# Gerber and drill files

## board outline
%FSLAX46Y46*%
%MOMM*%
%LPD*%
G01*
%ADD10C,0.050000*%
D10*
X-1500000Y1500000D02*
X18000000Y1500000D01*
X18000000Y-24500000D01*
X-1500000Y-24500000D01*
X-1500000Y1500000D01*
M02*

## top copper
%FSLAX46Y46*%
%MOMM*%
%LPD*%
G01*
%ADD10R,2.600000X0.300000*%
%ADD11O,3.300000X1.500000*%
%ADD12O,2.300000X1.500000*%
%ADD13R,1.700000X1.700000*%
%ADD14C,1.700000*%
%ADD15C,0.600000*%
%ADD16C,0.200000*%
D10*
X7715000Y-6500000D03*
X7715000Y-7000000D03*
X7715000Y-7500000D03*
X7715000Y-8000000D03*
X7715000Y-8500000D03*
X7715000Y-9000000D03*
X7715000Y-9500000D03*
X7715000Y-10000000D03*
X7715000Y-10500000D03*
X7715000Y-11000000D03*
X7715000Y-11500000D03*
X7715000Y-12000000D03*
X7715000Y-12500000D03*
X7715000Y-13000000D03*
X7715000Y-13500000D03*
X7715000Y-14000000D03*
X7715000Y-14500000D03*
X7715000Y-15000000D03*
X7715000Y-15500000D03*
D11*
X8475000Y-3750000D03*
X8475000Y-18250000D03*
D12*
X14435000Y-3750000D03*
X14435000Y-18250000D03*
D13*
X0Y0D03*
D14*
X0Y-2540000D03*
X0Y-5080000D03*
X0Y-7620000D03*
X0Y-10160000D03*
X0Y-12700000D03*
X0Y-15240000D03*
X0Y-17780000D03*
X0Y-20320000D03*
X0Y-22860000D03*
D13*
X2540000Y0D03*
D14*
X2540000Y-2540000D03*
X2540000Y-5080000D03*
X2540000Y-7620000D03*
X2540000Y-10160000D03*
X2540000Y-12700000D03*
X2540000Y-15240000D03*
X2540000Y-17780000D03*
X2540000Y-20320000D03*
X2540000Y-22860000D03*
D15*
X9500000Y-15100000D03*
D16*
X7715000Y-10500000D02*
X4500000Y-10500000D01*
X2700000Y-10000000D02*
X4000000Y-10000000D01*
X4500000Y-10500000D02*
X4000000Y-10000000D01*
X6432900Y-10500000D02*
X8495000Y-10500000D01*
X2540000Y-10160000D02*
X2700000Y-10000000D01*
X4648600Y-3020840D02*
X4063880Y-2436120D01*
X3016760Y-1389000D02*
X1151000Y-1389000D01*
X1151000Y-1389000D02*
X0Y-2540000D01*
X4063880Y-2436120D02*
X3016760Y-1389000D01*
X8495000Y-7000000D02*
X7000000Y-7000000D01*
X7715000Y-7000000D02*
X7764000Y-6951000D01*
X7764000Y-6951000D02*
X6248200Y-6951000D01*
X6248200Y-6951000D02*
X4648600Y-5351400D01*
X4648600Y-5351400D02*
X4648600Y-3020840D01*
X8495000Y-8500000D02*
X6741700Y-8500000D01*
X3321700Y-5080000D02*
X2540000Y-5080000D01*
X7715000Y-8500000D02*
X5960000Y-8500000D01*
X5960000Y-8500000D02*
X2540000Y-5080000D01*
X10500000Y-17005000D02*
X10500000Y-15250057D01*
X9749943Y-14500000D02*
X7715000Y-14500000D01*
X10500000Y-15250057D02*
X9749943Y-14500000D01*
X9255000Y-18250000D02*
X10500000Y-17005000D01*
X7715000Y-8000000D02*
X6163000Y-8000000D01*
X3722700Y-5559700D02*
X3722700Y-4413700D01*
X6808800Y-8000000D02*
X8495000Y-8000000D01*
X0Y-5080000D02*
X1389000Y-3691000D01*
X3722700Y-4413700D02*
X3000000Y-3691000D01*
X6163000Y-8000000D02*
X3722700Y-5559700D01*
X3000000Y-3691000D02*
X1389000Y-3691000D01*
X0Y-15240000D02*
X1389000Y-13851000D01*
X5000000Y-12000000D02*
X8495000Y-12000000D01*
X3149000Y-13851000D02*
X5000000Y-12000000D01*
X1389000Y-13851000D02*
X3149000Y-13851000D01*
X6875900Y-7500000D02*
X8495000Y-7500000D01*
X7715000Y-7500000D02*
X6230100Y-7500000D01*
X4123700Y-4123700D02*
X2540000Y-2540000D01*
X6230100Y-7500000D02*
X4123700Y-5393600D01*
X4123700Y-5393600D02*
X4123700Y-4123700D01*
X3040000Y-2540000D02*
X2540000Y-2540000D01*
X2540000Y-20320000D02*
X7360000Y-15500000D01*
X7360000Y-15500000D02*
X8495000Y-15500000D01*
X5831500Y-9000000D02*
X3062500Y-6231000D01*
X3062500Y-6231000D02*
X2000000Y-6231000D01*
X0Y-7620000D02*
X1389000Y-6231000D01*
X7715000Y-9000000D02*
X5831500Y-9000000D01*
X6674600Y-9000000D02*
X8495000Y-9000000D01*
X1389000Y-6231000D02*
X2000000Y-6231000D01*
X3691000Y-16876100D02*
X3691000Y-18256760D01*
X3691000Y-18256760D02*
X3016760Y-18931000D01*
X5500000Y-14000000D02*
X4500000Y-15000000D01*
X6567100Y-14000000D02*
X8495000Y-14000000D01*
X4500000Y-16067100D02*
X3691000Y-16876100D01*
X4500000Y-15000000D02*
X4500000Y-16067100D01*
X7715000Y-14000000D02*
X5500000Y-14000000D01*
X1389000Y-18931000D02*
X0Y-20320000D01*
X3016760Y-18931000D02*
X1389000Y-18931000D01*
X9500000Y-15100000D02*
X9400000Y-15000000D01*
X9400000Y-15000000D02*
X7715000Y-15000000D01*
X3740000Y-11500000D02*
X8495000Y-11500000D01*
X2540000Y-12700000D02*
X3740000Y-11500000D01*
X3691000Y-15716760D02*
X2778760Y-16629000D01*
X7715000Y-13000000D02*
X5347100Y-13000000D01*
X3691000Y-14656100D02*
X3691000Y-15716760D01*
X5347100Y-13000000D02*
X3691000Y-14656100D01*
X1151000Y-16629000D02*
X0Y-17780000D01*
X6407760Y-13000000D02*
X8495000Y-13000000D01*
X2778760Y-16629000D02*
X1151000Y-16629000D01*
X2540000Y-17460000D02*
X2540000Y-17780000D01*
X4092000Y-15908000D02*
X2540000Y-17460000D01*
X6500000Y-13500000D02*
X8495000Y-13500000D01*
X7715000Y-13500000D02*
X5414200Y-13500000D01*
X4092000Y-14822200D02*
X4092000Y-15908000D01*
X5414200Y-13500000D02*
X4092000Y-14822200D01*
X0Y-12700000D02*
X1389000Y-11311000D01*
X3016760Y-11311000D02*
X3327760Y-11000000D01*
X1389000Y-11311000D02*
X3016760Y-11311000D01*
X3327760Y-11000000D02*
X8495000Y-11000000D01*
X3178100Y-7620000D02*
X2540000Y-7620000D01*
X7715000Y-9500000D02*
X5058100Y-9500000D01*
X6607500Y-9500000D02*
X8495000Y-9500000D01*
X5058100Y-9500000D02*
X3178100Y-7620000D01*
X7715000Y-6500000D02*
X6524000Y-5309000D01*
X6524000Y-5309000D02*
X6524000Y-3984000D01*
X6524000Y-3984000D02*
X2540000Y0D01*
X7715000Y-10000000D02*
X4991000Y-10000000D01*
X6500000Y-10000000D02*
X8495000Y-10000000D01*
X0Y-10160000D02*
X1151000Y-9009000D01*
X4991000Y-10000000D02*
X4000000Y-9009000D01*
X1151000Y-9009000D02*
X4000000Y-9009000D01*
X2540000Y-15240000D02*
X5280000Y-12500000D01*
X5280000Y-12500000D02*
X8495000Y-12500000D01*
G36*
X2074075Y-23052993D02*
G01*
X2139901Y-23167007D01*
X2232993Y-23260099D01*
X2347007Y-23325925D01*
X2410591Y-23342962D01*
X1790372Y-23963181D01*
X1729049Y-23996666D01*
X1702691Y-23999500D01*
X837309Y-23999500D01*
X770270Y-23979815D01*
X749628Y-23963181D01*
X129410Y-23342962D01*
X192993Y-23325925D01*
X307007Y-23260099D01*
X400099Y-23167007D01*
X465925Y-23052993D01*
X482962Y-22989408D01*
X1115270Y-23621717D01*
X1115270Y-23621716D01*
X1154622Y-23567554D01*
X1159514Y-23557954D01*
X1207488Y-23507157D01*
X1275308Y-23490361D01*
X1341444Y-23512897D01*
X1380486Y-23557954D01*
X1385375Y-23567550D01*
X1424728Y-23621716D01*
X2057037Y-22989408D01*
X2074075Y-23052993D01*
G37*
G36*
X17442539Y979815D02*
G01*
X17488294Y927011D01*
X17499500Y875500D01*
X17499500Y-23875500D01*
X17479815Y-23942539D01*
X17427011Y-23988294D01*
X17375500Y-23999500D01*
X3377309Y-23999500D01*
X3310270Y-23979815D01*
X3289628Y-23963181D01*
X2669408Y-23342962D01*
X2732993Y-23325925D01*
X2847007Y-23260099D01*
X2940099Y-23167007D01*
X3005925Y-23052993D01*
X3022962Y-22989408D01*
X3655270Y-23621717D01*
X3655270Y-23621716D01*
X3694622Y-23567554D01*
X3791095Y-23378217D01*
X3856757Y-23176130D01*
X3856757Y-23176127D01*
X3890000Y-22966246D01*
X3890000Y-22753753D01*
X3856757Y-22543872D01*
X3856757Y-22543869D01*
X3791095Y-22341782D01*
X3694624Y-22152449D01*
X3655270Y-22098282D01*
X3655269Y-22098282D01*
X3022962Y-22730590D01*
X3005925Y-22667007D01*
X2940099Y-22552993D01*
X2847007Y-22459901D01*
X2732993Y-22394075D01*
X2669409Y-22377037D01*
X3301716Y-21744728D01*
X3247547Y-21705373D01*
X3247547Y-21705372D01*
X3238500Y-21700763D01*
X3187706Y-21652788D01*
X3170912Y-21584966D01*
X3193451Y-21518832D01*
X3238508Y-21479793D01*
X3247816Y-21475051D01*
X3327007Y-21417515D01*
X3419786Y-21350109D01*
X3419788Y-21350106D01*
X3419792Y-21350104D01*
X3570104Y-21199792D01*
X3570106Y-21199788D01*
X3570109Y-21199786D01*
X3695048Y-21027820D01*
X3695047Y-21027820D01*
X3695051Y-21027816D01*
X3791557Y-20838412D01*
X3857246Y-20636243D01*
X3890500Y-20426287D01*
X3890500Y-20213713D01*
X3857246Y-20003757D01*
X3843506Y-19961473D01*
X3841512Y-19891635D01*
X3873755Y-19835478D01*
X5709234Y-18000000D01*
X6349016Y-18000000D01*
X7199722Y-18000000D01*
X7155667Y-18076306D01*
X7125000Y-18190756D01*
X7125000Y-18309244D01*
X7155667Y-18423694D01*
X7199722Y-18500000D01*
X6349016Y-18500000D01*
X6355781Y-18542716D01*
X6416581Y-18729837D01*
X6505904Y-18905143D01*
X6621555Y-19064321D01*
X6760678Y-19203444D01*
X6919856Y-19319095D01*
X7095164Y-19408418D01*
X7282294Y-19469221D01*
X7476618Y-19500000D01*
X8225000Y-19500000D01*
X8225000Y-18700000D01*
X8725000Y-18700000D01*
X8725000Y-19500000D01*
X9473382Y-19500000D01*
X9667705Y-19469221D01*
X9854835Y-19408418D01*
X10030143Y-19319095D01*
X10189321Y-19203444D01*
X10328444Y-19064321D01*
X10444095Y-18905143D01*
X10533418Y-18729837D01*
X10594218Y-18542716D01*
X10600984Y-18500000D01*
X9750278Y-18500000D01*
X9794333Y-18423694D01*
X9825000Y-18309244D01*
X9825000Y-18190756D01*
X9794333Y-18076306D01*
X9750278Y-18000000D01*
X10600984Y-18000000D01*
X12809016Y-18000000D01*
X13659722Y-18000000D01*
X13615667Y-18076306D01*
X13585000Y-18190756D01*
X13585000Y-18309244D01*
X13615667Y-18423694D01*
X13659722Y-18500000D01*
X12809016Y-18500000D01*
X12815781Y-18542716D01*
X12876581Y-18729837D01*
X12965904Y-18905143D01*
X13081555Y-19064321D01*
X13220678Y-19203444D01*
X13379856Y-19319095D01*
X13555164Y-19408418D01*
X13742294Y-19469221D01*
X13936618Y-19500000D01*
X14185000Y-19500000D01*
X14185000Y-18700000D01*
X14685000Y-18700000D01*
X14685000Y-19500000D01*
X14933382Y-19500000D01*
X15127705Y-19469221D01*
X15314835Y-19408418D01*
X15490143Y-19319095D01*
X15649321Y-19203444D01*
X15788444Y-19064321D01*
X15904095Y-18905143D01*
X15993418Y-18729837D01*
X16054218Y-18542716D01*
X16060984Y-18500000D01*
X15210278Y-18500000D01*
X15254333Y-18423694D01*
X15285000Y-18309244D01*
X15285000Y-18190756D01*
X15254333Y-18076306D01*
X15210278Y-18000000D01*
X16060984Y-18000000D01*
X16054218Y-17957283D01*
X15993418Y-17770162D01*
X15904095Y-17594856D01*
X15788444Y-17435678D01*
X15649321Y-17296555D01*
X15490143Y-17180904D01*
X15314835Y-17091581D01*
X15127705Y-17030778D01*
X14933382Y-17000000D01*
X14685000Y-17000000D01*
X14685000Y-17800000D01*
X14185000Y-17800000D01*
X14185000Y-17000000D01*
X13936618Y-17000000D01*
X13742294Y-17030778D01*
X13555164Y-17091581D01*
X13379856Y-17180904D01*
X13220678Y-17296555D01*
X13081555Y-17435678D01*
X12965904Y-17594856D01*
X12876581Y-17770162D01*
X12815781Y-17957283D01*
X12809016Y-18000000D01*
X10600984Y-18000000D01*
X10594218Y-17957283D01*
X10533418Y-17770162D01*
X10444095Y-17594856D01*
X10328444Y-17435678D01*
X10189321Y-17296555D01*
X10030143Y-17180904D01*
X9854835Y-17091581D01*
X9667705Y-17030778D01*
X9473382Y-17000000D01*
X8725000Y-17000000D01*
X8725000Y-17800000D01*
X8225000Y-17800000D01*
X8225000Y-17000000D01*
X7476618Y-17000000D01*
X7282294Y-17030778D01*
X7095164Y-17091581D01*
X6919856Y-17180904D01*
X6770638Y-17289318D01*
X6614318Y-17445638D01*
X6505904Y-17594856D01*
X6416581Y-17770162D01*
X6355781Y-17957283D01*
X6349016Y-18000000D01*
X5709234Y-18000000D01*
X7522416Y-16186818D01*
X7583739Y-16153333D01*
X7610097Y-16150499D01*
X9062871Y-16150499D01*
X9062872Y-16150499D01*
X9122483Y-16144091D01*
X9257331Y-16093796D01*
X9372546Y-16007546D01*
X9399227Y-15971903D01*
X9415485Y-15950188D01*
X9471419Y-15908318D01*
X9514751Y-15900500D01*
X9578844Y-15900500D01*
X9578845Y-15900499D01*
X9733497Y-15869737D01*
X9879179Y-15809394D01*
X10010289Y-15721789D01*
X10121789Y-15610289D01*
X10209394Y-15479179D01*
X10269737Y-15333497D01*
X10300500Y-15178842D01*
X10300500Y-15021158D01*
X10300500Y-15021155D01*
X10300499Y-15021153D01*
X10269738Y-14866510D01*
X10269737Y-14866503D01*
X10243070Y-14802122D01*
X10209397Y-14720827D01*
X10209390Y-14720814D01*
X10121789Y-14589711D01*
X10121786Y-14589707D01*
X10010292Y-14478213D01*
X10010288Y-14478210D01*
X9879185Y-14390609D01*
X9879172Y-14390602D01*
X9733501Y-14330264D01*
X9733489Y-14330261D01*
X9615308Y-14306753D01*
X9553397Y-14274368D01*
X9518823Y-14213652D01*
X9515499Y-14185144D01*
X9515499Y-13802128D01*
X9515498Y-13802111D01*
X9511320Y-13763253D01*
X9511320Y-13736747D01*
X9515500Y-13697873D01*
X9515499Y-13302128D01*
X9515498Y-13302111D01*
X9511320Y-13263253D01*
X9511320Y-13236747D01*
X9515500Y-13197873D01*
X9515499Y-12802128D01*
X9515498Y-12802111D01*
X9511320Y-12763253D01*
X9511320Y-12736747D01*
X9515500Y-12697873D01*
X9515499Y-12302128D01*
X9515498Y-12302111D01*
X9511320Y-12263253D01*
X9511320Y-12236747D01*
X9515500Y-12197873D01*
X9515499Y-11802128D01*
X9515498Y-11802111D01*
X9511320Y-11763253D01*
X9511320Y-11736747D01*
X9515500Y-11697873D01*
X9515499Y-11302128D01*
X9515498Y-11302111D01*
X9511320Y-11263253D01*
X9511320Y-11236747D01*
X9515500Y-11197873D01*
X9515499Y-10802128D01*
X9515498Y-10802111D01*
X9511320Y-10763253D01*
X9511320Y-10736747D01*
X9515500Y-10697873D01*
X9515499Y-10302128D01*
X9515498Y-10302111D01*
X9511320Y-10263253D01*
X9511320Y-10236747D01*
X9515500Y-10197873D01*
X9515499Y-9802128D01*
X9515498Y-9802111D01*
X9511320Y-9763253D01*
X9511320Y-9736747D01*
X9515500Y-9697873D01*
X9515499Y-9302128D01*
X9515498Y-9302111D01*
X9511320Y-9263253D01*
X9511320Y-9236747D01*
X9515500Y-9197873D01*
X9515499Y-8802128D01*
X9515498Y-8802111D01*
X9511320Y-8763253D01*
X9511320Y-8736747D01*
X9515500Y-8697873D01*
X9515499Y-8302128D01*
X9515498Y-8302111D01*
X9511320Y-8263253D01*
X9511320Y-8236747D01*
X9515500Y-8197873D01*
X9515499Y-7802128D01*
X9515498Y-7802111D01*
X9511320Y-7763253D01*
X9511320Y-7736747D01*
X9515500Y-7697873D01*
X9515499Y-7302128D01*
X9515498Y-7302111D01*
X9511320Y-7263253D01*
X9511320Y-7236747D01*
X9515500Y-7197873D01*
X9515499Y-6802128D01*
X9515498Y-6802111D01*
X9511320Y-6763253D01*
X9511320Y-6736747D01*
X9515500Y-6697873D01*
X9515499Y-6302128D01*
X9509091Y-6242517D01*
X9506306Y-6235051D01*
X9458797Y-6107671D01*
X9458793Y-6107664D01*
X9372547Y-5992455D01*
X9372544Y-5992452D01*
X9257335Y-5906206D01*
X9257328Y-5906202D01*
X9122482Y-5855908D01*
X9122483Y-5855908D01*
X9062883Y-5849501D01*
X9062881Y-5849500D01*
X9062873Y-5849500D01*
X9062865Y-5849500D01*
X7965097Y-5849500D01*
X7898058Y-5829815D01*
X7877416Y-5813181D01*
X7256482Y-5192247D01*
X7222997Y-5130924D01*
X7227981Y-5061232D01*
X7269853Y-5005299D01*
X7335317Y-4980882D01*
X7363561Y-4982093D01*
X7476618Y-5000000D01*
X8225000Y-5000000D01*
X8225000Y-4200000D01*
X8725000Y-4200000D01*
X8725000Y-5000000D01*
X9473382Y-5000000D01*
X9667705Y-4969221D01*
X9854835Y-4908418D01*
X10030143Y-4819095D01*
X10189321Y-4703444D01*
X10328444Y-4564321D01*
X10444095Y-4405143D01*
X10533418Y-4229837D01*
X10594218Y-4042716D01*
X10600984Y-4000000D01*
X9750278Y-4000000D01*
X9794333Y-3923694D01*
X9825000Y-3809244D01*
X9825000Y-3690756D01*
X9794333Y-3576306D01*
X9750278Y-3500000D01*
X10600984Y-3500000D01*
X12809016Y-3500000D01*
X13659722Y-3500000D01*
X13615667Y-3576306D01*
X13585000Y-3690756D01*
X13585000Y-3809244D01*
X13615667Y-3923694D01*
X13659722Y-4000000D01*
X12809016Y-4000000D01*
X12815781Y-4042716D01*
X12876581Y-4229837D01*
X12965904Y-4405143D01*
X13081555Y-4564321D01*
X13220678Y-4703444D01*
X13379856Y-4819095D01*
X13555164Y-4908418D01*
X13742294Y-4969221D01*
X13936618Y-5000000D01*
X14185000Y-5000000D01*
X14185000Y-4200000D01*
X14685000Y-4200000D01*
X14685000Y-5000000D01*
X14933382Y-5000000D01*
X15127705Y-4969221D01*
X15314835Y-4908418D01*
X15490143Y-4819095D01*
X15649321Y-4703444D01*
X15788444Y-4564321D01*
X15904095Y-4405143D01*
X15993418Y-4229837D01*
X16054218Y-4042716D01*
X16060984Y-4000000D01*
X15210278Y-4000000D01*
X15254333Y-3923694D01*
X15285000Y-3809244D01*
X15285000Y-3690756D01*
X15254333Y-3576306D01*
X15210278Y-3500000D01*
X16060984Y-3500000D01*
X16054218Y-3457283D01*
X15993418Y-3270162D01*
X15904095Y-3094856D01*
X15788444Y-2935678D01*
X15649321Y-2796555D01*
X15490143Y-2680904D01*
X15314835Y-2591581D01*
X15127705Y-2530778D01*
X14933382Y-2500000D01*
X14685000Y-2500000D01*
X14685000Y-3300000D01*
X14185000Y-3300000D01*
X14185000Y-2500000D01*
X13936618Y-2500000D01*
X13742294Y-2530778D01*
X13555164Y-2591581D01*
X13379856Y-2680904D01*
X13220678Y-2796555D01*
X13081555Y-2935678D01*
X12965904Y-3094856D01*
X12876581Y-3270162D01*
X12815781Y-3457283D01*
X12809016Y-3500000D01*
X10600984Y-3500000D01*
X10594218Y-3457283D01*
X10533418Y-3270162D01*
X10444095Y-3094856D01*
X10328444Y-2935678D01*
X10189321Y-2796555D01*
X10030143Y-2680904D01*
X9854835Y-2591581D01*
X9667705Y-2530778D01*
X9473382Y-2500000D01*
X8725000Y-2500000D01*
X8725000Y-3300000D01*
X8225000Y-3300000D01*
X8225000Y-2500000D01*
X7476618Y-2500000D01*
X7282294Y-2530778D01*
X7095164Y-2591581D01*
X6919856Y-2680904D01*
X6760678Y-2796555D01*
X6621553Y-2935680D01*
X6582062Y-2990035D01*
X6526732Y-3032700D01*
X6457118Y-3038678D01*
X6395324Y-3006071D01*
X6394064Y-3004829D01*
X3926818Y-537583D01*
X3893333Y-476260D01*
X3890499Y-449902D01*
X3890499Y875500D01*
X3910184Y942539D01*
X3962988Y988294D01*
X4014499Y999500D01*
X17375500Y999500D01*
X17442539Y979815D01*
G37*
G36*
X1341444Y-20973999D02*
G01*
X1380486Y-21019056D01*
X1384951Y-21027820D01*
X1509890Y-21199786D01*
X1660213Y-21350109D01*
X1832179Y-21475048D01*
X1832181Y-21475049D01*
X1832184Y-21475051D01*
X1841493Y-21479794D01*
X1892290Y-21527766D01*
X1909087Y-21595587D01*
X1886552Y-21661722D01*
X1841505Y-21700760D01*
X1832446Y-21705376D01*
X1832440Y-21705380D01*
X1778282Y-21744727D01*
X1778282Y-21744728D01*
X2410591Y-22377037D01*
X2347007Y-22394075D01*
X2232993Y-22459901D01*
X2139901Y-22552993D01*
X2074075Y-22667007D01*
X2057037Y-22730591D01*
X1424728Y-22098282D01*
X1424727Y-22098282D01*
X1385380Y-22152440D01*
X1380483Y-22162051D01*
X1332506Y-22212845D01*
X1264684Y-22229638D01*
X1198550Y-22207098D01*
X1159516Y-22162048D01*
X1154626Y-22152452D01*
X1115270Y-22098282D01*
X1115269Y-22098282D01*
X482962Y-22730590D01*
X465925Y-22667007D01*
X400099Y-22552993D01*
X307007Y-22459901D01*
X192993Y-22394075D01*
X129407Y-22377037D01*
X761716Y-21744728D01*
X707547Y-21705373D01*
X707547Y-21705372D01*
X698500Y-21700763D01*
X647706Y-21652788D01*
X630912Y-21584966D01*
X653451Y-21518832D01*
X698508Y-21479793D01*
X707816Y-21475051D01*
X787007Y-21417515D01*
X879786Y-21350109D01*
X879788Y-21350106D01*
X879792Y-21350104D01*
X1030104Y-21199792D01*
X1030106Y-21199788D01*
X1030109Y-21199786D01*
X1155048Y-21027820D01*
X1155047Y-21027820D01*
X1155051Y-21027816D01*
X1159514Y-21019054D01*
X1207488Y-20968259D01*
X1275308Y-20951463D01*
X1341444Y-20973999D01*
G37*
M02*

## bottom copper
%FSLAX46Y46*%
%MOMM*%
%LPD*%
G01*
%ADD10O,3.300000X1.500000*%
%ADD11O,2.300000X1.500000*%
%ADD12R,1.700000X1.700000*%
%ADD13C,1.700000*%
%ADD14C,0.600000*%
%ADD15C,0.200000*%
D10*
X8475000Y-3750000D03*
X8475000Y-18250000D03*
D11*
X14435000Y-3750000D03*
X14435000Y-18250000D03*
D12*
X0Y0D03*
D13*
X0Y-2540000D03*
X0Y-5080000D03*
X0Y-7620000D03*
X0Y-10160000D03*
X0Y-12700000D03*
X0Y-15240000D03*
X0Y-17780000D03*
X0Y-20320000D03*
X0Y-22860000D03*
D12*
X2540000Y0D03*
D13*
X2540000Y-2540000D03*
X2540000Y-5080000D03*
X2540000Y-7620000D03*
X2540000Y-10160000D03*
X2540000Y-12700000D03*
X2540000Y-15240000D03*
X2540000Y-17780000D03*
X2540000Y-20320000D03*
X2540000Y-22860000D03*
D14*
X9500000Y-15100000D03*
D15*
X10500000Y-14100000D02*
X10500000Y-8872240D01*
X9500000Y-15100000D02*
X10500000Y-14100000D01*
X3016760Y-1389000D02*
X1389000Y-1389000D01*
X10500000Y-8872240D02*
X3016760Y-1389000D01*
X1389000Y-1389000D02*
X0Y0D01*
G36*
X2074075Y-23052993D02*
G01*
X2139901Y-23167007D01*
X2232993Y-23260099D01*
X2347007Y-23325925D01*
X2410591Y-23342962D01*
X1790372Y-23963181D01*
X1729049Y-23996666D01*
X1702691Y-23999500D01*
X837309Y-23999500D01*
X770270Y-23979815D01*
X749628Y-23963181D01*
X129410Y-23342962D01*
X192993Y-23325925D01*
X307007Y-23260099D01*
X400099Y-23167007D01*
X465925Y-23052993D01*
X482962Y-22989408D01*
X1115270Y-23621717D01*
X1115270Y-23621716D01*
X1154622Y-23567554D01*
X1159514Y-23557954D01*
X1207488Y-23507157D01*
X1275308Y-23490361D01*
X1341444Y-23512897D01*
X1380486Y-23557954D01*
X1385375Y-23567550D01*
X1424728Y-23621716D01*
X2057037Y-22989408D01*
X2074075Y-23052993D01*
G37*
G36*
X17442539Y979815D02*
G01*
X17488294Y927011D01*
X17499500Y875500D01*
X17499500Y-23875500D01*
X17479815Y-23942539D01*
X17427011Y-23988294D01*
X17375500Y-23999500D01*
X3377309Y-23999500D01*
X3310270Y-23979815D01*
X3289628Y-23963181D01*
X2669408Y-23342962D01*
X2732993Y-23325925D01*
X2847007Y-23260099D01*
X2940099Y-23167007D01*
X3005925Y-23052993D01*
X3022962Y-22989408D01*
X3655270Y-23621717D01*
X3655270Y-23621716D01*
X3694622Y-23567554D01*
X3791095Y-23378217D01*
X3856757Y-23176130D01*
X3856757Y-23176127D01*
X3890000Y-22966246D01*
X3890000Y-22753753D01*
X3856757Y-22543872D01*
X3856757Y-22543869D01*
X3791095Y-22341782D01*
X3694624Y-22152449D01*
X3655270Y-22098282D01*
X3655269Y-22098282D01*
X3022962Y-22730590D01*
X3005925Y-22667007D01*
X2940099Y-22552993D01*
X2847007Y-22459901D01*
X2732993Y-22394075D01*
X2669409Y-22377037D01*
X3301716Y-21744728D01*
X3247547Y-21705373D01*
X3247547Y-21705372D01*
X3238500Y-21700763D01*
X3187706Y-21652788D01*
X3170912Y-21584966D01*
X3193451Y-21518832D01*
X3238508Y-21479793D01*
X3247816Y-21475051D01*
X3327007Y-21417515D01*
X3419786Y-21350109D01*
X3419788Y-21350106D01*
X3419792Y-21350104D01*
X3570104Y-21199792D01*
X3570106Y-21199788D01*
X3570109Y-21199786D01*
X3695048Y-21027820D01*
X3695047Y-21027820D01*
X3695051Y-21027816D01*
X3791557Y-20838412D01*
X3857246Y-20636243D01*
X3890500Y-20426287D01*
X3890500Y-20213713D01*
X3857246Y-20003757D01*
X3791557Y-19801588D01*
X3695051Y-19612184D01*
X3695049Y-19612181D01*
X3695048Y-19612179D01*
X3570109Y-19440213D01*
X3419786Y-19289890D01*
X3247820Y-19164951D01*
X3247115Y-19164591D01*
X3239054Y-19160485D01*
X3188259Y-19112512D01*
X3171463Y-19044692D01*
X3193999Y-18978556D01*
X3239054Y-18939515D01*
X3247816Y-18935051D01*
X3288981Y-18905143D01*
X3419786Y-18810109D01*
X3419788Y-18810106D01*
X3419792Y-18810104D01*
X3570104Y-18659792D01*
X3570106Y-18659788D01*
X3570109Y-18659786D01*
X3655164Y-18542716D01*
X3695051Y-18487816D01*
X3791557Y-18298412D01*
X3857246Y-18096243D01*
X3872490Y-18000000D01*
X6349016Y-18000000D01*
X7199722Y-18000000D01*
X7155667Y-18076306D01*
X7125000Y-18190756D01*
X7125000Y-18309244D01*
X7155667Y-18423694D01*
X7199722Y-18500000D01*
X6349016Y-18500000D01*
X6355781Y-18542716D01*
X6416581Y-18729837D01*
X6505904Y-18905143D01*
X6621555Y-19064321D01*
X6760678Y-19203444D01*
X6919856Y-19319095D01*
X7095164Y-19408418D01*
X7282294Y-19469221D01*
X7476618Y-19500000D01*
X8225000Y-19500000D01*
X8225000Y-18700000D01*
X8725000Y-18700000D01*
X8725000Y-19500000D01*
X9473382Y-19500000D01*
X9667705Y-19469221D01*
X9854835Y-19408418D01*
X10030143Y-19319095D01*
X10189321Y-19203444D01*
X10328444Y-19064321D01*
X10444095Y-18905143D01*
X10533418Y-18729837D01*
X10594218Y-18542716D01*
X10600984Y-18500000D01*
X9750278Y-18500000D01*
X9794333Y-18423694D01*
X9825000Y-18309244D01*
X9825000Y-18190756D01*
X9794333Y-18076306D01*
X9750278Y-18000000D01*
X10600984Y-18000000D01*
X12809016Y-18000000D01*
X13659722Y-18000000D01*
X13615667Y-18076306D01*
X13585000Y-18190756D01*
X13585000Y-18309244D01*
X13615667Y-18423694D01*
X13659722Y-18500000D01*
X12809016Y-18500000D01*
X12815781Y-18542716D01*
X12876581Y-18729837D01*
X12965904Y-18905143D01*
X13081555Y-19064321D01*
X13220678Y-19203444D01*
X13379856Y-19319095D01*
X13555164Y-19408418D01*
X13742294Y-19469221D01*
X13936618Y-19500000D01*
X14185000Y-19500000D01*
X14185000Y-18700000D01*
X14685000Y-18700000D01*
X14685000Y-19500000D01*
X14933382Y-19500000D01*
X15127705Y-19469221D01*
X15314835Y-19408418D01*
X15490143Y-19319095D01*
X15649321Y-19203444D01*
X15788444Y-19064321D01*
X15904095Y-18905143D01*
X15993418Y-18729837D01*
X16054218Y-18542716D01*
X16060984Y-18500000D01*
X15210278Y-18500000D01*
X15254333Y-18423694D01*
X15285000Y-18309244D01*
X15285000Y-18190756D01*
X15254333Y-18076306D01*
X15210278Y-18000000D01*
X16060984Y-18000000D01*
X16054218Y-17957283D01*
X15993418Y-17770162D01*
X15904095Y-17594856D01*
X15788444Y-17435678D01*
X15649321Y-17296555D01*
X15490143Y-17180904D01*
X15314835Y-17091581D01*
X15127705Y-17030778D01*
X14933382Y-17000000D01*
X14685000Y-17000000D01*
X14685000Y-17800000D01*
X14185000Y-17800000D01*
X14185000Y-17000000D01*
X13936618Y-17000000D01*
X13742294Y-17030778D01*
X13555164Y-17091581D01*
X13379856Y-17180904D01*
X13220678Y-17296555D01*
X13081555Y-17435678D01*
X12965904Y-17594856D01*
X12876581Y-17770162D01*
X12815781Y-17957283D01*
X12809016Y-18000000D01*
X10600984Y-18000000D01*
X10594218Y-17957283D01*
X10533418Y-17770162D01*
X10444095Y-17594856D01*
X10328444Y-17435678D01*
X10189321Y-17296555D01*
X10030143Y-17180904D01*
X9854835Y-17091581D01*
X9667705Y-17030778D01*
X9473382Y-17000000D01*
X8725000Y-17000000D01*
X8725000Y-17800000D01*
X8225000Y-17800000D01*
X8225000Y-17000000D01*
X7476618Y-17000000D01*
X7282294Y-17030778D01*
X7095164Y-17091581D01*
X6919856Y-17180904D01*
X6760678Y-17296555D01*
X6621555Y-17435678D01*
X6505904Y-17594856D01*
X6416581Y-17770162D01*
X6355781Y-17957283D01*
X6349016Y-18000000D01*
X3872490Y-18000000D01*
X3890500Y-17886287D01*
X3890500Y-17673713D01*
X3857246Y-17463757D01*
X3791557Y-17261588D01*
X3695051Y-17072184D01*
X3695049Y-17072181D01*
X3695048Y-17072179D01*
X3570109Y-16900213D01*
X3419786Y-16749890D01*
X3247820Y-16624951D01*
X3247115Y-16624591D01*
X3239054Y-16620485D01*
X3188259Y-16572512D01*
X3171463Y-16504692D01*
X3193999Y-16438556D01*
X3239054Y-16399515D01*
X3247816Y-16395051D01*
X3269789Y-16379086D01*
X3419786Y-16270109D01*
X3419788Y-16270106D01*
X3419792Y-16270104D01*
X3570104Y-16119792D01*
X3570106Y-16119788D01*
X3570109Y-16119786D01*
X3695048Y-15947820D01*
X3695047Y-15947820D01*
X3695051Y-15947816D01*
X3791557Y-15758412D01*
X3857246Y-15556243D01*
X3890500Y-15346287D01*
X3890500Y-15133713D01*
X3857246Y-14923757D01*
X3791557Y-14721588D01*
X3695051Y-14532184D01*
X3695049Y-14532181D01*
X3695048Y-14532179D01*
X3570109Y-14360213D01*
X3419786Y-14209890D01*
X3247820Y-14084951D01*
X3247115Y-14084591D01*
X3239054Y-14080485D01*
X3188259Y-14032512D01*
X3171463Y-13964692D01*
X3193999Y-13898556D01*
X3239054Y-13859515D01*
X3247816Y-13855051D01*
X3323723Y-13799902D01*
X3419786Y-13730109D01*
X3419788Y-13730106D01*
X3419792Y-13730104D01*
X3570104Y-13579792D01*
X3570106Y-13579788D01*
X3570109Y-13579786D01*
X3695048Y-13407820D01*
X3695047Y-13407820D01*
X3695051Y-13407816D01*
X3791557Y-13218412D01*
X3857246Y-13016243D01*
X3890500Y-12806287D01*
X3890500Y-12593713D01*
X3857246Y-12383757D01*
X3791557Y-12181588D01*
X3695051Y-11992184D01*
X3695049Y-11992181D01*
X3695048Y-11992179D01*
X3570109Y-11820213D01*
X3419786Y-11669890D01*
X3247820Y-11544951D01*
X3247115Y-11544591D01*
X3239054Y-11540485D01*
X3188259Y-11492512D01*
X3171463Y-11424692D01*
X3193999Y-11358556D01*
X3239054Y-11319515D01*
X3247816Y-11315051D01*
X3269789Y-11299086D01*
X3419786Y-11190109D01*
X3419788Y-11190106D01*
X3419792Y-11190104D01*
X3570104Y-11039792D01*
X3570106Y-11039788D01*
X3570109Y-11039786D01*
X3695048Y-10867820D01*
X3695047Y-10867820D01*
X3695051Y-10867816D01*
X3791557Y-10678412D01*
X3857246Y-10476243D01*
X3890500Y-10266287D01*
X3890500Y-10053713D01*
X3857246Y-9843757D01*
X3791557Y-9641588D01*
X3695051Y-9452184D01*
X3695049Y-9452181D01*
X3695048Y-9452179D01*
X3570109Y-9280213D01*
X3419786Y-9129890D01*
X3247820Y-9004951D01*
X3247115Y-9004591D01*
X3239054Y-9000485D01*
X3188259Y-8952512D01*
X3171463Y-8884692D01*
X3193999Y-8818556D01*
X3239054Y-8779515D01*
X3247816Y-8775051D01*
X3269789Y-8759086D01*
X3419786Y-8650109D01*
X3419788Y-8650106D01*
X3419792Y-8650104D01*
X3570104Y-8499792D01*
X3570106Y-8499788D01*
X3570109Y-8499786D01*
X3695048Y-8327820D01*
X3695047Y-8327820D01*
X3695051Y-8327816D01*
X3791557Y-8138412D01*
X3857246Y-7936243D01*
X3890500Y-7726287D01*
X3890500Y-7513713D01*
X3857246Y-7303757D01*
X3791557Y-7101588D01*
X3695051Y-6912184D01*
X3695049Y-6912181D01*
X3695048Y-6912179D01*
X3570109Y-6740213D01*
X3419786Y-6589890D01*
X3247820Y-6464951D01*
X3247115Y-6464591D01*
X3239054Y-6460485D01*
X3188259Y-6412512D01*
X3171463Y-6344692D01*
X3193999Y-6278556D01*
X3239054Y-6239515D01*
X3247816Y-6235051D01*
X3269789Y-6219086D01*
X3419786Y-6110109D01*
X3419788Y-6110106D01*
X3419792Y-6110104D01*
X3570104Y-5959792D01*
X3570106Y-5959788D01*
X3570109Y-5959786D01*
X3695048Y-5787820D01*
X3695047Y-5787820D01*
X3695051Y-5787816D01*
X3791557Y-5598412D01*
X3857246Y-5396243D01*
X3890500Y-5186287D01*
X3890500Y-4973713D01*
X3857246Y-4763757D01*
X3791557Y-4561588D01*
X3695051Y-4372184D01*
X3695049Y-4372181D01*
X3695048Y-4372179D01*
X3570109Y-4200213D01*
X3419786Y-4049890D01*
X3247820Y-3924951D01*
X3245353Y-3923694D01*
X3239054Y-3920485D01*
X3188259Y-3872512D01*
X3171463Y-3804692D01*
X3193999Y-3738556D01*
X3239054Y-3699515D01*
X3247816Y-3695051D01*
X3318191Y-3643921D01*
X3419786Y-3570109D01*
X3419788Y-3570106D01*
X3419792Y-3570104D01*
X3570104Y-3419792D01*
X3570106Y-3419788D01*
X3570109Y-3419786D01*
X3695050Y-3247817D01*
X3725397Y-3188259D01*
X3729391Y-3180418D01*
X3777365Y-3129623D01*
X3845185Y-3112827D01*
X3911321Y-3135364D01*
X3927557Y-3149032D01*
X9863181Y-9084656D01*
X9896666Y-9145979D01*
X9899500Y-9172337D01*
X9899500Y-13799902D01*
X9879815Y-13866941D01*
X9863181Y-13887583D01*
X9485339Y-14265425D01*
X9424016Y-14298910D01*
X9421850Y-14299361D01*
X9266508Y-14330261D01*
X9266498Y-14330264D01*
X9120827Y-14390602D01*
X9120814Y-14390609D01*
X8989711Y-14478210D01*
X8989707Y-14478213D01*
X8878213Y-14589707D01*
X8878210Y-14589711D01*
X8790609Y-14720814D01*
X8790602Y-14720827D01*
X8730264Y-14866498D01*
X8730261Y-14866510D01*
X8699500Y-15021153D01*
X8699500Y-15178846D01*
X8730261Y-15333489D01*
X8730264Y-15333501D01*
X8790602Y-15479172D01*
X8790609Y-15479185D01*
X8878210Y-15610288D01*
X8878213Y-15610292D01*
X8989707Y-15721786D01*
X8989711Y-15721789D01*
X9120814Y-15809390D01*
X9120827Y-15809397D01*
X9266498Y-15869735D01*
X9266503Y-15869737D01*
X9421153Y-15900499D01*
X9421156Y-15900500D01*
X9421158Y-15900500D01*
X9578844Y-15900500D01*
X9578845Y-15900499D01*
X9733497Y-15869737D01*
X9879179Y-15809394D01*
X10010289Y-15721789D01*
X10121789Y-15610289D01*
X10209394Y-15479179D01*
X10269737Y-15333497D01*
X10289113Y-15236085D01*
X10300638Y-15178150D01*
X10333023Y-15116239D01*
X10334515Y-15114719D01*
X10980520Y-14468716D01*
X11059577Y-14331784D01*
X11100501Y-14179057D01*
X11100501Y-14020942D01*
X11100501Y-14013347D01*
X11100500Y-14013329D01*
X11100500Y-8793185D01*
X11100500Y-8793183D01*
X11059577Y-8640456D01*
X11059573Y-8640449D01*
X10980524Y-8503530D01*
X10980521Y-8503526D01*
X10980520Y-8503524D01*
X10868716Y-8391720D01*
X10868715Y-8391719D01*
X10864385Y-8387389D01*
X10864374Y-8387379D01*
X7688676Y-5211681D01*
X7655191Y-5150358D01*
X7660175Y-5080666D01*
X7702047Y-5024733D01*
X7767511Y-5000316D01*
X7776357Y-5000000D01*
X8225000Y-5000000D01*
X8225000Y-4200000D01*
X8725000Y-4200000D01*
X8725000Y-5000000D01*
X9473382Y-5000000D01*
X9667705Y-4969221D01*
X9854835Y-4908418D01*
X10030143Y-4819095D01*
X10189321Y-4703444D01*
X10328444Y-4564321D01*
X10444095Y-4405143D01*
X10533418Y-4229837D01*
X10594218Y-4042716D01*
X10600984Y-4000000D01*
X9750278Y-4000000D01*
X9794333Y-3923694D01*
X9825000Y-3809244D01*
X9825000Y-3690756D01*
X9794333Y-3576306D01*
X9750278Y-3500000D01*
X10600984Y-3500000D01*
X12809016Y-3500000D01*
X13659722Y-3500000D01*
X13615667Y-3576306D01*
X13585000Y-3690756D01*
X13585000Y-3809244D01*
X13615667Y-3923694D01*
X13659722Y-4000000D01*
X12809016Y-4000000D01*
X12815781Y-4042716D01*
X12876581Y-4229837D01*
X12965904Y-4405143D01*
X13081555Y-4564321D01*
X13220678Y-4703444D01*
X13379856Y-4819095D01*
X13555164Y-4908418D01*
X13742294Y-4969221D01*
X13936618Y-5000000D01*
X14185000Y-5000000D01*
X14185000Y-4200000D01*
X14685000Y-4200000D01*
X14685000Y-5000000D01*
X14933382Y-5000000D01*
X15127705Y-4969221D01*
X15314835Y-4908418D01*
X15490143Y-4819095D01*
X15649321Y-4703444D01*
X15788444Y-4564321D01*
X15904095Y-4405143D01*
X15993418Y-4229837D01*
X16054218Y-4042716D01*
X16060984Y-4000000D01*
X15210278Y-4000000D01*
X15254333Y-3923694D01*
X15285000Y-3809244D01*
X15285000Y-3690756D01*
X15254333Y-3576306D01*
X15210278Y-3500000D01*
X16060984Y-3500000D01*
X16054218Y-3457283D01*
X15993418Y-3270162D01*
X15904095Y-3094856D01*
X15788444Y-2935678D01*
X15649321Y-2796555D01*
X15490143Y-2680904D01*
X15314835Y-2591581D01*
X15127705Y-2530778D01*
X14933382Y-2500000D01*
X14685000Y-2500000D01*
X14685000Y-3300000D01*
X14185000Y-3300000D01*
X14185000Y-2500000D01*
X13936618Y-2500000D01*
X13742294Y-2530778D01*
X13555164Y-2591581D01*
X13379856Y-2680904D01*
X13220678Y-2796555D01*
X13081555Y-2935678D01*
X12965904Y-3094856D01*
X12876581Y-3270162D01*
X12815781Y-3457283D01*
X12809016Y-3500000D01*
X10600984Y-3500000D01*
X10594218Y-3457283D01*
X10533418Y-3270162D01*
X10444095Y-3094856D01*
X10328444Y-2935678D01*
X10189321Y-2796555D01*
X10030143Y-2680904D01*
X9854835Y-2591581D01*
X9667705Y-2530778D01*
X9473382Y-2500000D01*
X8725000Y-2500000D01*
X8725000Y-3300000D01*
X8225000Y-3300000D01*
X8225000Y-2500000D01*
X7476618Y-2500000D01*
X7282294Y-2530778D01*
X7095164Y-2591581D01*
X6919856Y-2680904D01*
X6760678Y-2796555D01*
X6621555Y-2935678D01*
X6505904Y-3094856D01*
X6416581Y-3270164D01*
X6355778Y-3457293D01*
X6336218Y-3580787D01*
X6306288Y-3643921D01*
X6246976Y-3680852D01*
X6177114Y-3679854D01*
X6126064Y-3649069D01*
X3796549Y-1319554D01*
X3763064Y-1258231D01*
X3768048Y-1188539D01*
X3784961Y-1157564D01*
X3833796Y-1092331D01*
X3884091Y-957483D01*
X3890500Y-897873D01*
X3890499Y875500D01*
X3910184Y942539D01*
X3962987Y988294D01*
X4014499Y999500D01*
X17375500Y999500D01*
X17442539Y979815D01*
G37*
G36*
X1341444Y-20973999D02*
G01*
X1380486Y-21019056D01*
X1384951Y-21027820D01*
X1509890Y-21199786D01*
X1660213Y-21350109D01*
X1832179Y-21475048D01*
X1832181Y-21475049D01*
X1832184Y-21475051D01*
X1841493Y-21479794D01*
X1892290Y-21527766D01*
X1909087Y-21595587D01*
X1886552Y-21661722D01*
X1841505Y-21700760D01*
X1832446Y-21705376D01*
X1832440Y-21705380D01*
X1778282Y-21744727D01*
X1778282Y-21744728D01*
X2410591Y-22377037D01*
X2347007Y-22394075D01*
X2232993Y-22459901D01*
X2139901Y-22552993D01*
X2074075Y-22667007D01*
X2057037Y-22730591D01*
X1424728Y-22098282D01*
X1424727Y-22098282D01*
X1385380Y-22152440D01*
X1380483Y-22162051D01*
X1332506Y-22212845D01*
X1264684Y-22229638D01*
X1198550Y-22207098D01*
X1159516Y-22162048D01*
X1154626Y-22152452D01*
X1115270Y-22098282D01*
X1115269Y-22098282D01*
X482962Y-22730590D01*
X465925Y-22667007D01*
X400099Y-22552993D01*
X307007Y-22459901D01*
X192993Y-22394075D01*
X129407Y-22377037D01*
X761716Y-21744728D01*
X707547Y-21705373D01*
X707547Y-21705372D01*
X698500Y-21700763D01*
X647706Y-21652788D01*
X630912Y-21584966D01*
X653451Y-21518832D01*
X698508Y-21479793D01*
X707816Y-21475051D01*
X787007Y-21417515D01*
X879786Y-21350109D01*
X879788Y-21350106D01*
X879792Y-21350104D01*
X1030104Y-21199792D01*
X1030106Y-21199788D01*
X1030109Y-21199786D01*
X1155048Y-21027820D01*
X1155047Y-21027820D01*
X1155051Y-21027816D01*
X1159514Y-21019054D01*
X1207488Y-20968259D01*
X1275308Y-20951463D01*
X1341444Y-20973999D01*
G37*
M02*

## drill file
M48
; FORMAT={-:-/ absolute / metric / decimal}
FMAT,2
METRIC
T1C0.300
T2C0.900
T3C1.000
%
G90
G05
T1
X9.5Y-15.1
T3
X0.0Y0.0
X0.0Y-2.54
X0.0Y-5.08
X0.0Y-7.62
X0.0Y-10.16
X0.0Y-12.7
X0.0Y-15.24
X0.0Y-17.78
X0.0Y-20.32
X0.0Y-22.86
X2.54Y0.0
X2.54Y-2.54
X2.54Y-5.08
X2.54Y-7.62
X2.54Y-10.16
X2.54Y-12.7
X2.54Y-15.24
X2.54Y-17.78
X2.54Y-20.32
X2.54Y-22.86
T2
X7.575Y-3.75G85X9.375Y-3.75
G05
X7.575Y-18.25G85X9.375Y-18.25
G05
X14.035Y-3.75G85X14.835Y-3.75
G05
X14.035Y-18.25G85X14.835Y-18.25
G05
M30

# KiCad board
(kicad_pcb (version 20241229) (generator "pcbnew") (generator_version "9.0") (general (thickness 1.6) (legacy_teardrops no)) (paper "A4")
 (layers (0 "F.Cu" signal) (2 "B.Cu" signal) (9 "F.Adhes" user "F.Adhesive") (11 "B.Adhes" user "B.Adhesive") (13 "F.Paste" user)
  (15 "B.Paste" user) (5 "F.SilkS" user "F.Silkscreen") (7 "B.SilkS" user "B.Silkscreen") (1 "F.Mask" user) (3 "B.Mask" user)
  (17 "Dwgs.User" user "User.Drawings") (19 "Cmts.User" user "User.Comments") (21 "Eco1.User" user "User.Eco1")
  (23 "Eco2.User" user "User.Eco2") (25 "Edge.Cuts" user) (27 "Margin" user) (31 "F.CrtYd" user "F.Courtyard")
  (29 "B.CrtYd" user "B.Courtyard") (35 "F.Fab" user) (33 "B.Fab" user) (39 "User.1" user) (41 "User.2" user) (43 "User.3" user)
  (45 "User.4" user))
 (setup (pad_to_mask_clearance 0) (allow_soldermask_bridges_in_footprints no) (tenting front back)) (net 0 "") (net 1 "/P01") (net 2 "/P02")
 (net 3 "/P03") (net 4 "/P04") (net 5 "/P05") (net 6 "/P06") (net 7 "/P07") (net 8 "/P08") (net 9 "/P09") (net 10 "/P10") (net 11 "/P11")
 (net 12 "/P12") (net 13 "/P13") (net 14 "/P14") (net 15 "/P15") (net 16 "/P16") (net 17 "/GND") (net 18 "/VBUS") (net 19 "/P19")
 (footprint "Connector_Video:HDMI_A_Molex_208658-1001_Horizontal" (layer "F.Cu") (at 11 11)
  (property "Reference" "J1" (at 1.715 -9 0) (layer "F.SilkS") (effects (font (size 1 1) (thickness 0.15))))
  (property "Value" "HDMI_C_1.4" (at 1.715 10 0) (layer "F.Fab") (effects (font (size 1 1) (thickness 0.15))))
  (pad "1" smd rect (at -3.285 -4.5) (size 2.6 0.3) (layers "F.Cu" "F.Mask" "F.Paste") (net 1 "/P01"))
  (pad "2" smd rect (at -3.285 -4) (size 2.6 0.3) (layers "F.Cu" "F.Mask" "F.Paste") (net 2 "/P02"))
  (pad "3" smd rect (at -3.285 -3.5) (size 2.6 0.3) (layers "F.Cu" "F.Mask" "F.Paste") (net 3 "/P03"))
  (pad "4" smd rect (at -3.285 -3) (size 2.6 0.3) (layers "F.Cu" "F.Mask" "F.Paste") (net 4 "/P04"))
  (pad "5" smd rect (at -3.285 -2.5) (size 2.6 0.3) (layers "F.Cu" "F.Mask" "F.Paste") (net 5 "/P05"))
  (pad "6" smd rect (at -3.285 -2) (size 2.6 0.3) (layers "F.Cu" "F.Mask" "F.Paste") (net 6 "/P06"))
  (pad "7" smd rect (at -3.285 -1.5) (size 2.6 0.3) (layers "F.Cu" "F.Mask" "F.Paste") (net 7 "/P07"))
  (pad "8" smd rect (at -3.285 -1) (size 2.6 0.3) (layers "F.Cu" "F.Mask" "F.Paste") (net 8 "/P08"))
  (pad "9" smd rect (at -3.285 -0.5) (size 2.6 0.3) (layers "F.Cu" "F.Mask" "F.Paste") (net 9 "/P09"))
  (pad "10" smd rect (at -3.285 0) (size 2.6 0.3) (layers "F.Cu" "F.Mask" "F.Paste") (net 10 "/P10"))
  (pad "11" smd rect (at -3.285 0.5) (size 2.6 0.3) (layers "F.Cu" "F.Mask" "F.Paste") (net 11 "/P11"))
  (pad "12" smd rect (at -3.285 1) (size 2.6 0.3) (layers "F.Cu" "F.Mask" "F.Paste") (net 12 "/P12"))
  (pad "13" smd rect (at -3.285 1.5) (size 2.6 0.3) (layers "F.Cu" "F.Mask" "F.Paste") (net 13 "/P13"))
  (pad "14" smd rect (at -3.285 2) (size 2.6 0.3) (layers "F.Cu" "F.Mask" "F.Paste") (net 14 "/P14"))
  (pad "15" smd rect (at -3.285 2.5) (size 2.6 0.3) (layers "F.Cu" "F.Mask" "F.Paste") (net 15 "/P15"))
  (pad "16" smd rect (at -3.285 3) (size 2.6 0.3) (layers "F.Cu" "F.Mask" "F.Paste") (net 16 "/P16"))
  (pad "17" smd rect (at -3.285 3.5) (size 2.6 0.3) (layers "F.Cu" "F.Mask" "F.Paste") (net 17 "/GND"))
  (pad "18" smd rect (at -3.285 4) (size 2.6 0.3) (layers "F.Cu" "F.Mask" "F.Paste") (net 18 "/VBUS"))
  (pad "19" smd rect (at -3.285 4.5) (size 2.6 0.3) (layers "F.Cu" "F.Mask" "F.Paste") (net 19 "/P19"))
  (pad "SH" thru_hole oval (at -2.525 -7.25) (size 3.3 1.5) (drill oval 2.7 0.9) (layers "*.Cu" "*.Mask") (remove_unused_layers no)
   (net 17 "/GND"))
  (pad "SH" thru_hole oval (at -2.525 7.25) (size 3.3 1.5) (drill oval 2.7 0.9) (layers "*.Cu" "*.Mask") (remove_unused_layers no)
   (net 17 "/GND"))
  (pad "SH" thru_hole oval (at 3.435 -7.25) (size 2.3 1.5) (drill oval 1.7 0.9) (layers "*.Cu" "*.Mask") (remove_unused_layers no)
   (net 17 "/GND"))
  (pad "SH" thru_hole oval (at 3.435 7.25) (size 2.3 1.5) (drill oval 1.7 0.9) (layers "*.Cu" "*.Mask") (remove_unused_layers no)
   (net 17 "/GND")))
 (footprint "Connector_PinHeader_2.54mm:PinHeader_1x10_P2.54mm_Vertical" (layer "F.Cu") (at 0 0)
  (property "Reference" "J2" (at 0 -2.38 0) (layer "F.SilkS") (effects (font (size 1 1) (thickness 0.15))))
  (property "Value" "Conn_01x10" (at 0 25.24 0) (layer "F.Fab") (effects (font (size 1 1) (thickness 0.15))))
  (pad "1" thru_hole rect (at 0 0) (size 1.7 1.7) (drill 1) (layers "*.Cu" "*.Mask") (remove_unused_layers no) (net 18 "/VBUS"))
  (pad "2" thru_hole circle (at 0 2.54) (size 1.7 1.7) (drill 1) (layers "*.Cu" "*.Mask") (remove_unused_layers no) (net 2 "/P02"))
  (pad "3" thru_hole circle (at 0 5.08) (size 1.7 1.7) (drill 1) (layers "*.Cu" "*.Mask") (remove_unused_layers no) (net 4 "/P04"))
  (pad "4" thru_hole circle (at 0 7.62) (size 1.7 1.7) (drill 1) (layers "*.Cu" "*.Mask") (remove_unused_layers no) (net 6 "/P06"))
  (pad "5" thru_hole circle (at 0 10.16) (size 1.7 1.7) (drill 1) (layers "*.Cu" "*.Mask") (remove_unused_layers no) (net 8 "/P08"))
  (pad "6" thru_hole circle (at 0 12.7) (size 1.7 1.7) (drill 1) (layers "*.Cu" "*.Mask") (remove_unused_layers no) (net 10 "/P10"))
  (pad "7" thru_hole circle (at 0 15.24) (size 1.7 1.7) (drill 1) (layers "*.Cu" "*.Mask") (remove_unused_layers no) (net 12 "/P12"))
  (pad "8" thru_hole circle (at 0 17.78) (size 1.7 1.7) (drill 1) (layers "*.Cu" "*.Mask") (remove_unused_layers no) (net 14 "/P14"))
  (pad "9" thru_hole circle (at 0 20.32) (size 1.7 1.7) (drill 1) (layers "*.Cu" "*.Mask") (remove_unused_layers no) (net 16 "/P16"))
  (pad "10" thru_hole circle (at 0 22.86) (size 1.7 1.7) (drill 1) (layers "*.Cu" "*.Mask") (remove_unused_layers no) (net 17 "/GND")))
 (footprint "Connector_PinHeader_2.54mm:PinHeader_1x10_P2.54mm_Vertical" (layer "F.Cu") (at 2.54 0)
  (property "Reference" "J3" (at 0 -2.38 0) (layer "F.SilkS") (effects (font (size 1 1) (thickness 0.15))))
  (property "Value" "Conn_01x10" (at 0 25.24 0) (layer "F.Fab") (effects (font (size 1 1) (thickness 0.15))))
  (pad "1" thru_hole rect (at 0 0) (size 1.7 1.7) (drill 1) (layers "*.Cu" "*.Mask") (remove_unused_layers no) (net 1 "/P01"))
  (pad "2" thru_hole circle (at 0 2.54) (size 1.7 1.7) (drill 1) (layers "*.Cu" "*.Mask") (remove_unused_layers no) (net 3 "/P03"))
  (pad "3" thru_hole circle (at 0 5.08) (size 1.7 1.7) (drill 1) (layers "*.Cu" "*.Mask") (remove_unused_layers no) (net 5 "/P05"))
  (pad "4" thru_hole circle (at 0 7.62) (size 1.7 1.7) (drill 1) (layers "*.Cu" "*.Mask") (remove_unused_layers no) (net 7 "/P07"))
  (pad "5" thru_hole circle (at 0 10.16) (size 1.7 1.7) (drill 1) (layers "*.Cu" "*.Mask") (remove_unused_layers no) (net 9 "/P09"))
  (pad "6" thru_hole circle (at 0 12.7) (size 1.7 1.7) (drill 1) (layers "*.Cu" "*.Mask") (remove_unused_layers no) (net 11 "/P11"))
  (pad "7" thru_hole circle (at 0 15.24) (size 1.7 1.7) (drill 1) (layers "*.Cu" "*.Mask") (remove_unused_layers no) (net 13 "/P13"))
  (pad "8" thru_hole circle (at 0 17.78) (size 1.7 1.7) (drill 1) (layers "*.Cu" "*.Mask") (remove_unused_layers no) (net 15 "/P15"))
  (pad "9" thru_hole circle (at 0 20.32) (size 1.7 1.7) (drill 1) (layers "*.Cu" "*.Mask") (remove_unused_layers no) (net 19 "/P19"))
  (pad "10" thru_hole circle (at 0 22.86) (size 1.7 1.7) (drill 1) (layers "*.Cu" "*.Mask") (remove_unused_layers no) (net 17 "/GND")))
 (gr_rect (start -1.5 -1.5) (end 18 24.5) (stroke (width 0.05) (type default)) (fill no) (layer "Edge.Cuts"))
 (segment (start 7.715 10.5) (end 4.5 10.5) (width 0.2) (layer "F.Cu") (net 9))
 (segment (start 2.7 10) (end 4 10) (width 0.2) (layer "F.Cu") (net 9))
 (segment (start 4.5 10.5) (end 4 10) (width 0.2) (layer "F.Cu") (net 9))
 (segment (start 6.4329 10.5) (end 8.495 10.5) (width 0.2) (layer "F.Cu") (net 9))
 (segment (start 2.54 10.16) (end 2.7 10) (width 0.2) (layer "F.Cu") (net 9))
 (segment (start 4.6486 3.02084) (end 4.06388 2.43612) (width 0.2) (layer "F.Cu") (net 2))
 (segment (start 3.01676 1.389) (end 1.151 1.389) (width 0.2) (layer "F.Cu") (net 2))
 (segment (start 1.151 1.389) (end 0 2.54) (width 0.2) (layer "F.Cu") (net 2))
 (segment (start 4.06388 2.43612) (end 3.01676 1.389) (width 0.2) (layer "F.Cu") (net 2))
 (segment (start 8.495 7) (end 7 7) (width 0.2) (layer "F.Cu") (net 2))
 (segment (start 7.715 7) (end 7.764 6.951) (width 0.2) (layer "F.Cu") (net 2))
 (segment (start 7.764 6.951) (end 6.2482 6.951) (width 0.2) (layer "F.Cu") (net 2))
 (segment (start 6.2482 6.951) (end 4.6486 5.3514) (width 0.2) (layer "F.Cu") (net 2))
 (segment (start 4.6486 5.3514) (end 4.6486 3.02084) (width 0.2) (layer "F.Cu") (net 2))
 (segment (start 8.495 8.5) (end 6.7417 8.5) (width 0.2) (layer "F.Cu") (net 5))
 (segment (start 3.3217 5.08) (end 2.54 5.08) (width 0.2) (layer "F.Cu") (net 5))
 (segment (start 7.715 8.5) (end 5.96 8.5) (width 0.2) (layer "F.Cu") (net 5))
 (segment (start 5.96 8.5) (end 2.54 5.08) (width 0.2) (layer "F.Cu") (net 5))
 (segment (start 10.5 17.005) (end 10.5 15.250057) (width 0.2) (layer "F.Cu") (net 17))
 (segment (start 9.749943 14.5) (end 7.715 14.5) (width 0.2) (layer "F.Cu") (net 17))
 (segment (start 10.5 15.250057) (end 9.749943 14.5) (width 0.2) (layer "F.Cu") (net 17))
 (segment (start 9.255 18.25) (end 10.5 17.005) (width 0.2) (layer "F.Cu") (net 17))
 (segment (start 7.715 8) (end 6.163 8) (width 0.2) (layer "F.Cu") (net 4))
 (segment (start 3.7227 5.5597) (end 3.7227 4.4137) (width 0.2) (layer "F.Cu") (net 4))
 (segment (start 6.8088 8) (end 8.495 8) (width 0.2) (layer "F.Cu") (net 4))
 (segment (start 0 5.08) (end 1.389 3.691) (width 0.2) (layer "F.Cu") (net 4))
 (segment (start 3.7227 4.4137) (end 3 3.691) (width 0.2) (layer "F.Cu") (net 4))
 (segment (start 6.163 8) (end 3.7227 5.5597) (width 0.2) (layer "F.Cu") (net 4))
 (segment (start 3 3.691) (end 1.389 3.691) (width 0.2) (layer "F.Cu") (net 4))
 (segment (start 0 15.24) (end 1.389 13.851) (width 0.2) (layer "F.Cu") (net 12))
 (segment (start 5 12) (end 8.495 12) (width 0.2) (layer "F.Cu") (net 12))
 (segment (start 3.149 13.851) (end 5 12) (width 0.2) (layer "F.Cu") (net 12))
 (segment (start 1.389 13.851) (end 3.149 13.851) (width 0.2) (layer "F.Cu") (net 12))
 (segment (start 6.8759 7.5) (end 8.495 7.5) (width 0.2) (layer "F.Cu") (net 3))
 (segment (start 7.715 7.5) (end 6.2301 7.5) (width 0.2) (layer "F.Cu") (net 3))
 (segment (start 4.1237 4.1237) (end 2.54 2.54) (width 0.2) (layer "F.Cu") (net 3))
 (segment (start 6.2301 7.5) (end 4.1237 5.3936) (width 0.2) (layer "F.Cu") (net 3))
 (segment (start 4.1237 5.3936) (end 4.1237 4.1237) (width 0.2) (layer "F.Cu") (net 3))
 (segment (start 3.04 2.54) (end 2.54 2.54) (width 0.2) (layer "F.Cu") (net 3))
 (segment (start 2.54 20.32) (end 7.36 15.5) (width 0.2) (layer "F.Cu") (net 19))
 (segment (start 7.36 15.5) (end 8.495 15.5) (width 0.2) (layer "F.Cu") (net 19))
 (segment (start 5.8315 9) (end 3.0625 6.231) (width 0.2) (layer "F.Cu") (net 6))
 (segment (start 3.0625 6.231) (end 2 6.231) (width 0.2) (layer "F.Cu") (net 6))
 (segment (start 0 7.62) (end 1.389 6.231) (width 0.2) (layer "F.Cu") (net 6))
 (segment (start 7.715 9) (end 5.8315 9) (width 0.2) (layer "F.Cu") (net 6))
 (segment (start 6.6746 9) (end 8.495 9) (width 0.2) (layer "F.Cu") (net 6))
 (segment (start 1.389 6.231) (end 2 6.231) (width 0.2) (layer "F.Cu") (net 6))
 (segment (start 3.691 16.8761) (end 3.691 18.25676) (width 0.2) (layer "F.Cu") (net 16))
 (segment (start 3.691 18.25676) (end 3.01676 18.931) (width 0.2) (layer "F.Cu") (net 16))
 (segment (start 5.5 14) (end 4.5 15) (width 0.2) (layer "F.Cu") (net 16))
 (segment (start 6.5671 14) (end 8.495 14) (width 0.2) (layer "F.Cu") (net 16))
 (segment (start 4.5 16.0671) (end 3.691 16.8761) (width 0.2) (layer "F.Cu") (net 16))
 (segment (start 4.5 15) (end 4.5 16.0671) (width 0.2) (layer "F.Cu") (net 16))
 (segment (start 7.715 14) (end 5.5 14) (width 0.2) (layer "F.Cu") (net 16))
 (segment (start 1.389 18.931) (end 0 20.32) (width 0.2) (layer "F.Cu") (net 16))
 (segment (start 3.01676 18.931) (end 1.389 18.931) (width 0.2) (layer "F.Cu") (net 16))
 (segment (start 9.5 15.1) (end 9.4 15) (width 0.2) (layer "F.Cu") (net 18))
 (segment (start 9.4 15) (end 7.715 15) (width 0.2) (layer "F.Cu") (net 18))
 (via (at 9.5 15.1) (size 0.6) (drill 0.3) (layers "F.Cu" "B.Cu") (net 18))
 (segment (start 10.5 14.1) (end 10.5 8.87224) (width 0.2) (layer "B.Cu") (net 18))
 (segment (start 9.5 15.1) (end 10.5 14.1) (width 0.2) (layer "B.Cu") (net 18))
 (segment (start 3.01676 1.389) (end 1.389 1.389) (width 0.2) (layer "B.Cu") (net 18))
 (segment (start 10.5 8.87224) (end 3.01676 1.389) (width 0.2) (layer "B.Cu") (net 18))
 (segment (start 1.389 1.389) (end 0 0) (width 0.2) (layer "B.Cu") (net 18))
 (segment (start 3.74 11.5) (end 8.495 11.5) (width 0.2) (layer "F.Cu") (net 11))
 (segment (start 2.54 12.7) (end 3.74 11.5) (width 0.2) (layer "F.Cu") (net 11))
 (segment (start 3.691 15.71676) (end 2.77876 16.629) (width 0.2) (layer "F.Cu") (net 14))
 (segment (start 7.715 13) (end 5.3471 13) (width 0.2) (layer "F.Cu") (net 14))
 (segment (start 3.691 14.6561) (end 3.691 15.71676) (width 0.2) (layer "F.Cu") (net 14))
 (segment (start 5.3471 13) (end 3.691 14.6561) (width 0.2) (layer "F.Cu") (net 14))
 (segment (start 1.151 16.629) (end 0 17.78) (width 0.2) (layer "F.Cu") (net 14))
 (segment (start 6.40776 13) (end 8.495 13) (width 0.2) (layer "F.Cu") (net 14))
 (segment (start 2.77876 16.629) (end 1.151 16.629) (width 0.2) (layer "F.Cu") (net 14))
 (segment (start 2.54 17.46) (end 2.54 17.78) (width 0.2) (layer "F.Cu") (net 15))
 (segment (start 4.092 15.908) (end 2.54 17.46) (width 0.2) (layer "F.Cu") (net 15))
 (segment (start 6.5 13.5) (end 8.495 13.5) (width 0.2) (layer "F.Cu") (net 15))
 (segment (start 7.715 13.5) (end 5.4142 13.5) (width 0.2) (layer "F.Cu") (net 15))
 (segment (start 4.092 14.8222) (end 4.092 15.908) (width 0.2) (layer "F.Cu") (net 15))
 (segment (start 5.4142 13.5) (end 4.092 14.8222) (width 0.2) (layer "F.Cu") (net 15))
 (segment (start 0 12.7) (end 1.389 11.311) (width 0.2) (layer "F.Cu") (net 10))
 (segment (start 3.01676 11.311) (end 3.32776 11) (width 0.2) (layer "F.Cu") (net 10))
 (segment (start 1.389 11.311) (end 3.01676 11.311) (width 0.2) (layer "F.Cu") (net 10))
 (segment (start 3.32776 11) (end 8.495 11) (width 0.2) (layer "F.Cu") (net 10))
 (segment (start 3.1781 7.62) (end 2.54 7.62) (width 0.2) (layer "F.Cu") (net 7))
 (segment (start 7.715 9.5) (end 5.0581 9.5) (width 0.2) (layer "F.Cu") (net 7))
 (segment (start 6.6075 9.5) (end 8.495 9.5) (width 0.2) (layer "F.Cu") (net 7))
 (segment (start 5.0581 9.5) (end 3.1781 7.62) (width 0.2) (layer "F.Cu") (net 7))
 (segment (start 7.715 6.5) (end 6.524 5.309) (width 0.2) (layer "F.Cu") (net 1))
 (segment (start 6.524 5.309) (end 6.524 3.984) (width 0.2) (layer "F.Cu") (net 1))
 (segment (start 6.524 3.984) (end 2.54 0) (width 0.2) (layer "F.Cu") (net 1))
 (segment (start 7.715 10) (end 4.991 10) (width 0.2) (layer "F.Cu") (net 8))
 (segment (start 6.5 10) (end 8.495 10) (width 0.2) (layer "F.Cu") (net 8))
 (segment (start 0 10.16) (end 1.151 9.009) (width 0.2) (layer "F.Cu") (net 8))
 (segment (start 4.991 10) (end 4 9.009) (width 0.2) (layer "F.Cu") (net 8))
 (segment (start 1.151 9.009) (end 4 9.009) (width 0.2) (layer "F.Cu") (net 8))
 (segment (start 2.54 15.24) (end 5.28 12.5) (width 0.2) (layer "F.Cu") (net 13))
 (segment (start 5.28 12.5) (end 8.495 12.5) (width 0.2) (layer "F.Cu") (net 13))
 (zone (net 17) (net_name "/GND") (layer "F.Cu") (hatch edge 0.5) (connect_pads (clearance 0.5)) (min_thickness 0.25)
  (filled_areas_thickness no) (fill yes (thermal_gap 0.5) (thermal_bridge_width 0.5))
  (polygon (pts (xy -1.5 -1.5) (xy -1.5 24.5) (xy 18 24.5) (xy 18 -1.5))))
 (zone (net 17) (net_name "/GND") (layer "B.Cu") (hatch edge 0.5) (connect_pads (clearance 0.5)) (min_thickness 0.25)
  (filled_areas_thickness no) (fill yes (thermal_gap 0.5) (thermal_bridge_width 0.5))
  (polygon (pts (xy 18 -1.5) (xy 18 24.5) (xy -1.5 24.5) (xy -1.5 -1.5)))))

